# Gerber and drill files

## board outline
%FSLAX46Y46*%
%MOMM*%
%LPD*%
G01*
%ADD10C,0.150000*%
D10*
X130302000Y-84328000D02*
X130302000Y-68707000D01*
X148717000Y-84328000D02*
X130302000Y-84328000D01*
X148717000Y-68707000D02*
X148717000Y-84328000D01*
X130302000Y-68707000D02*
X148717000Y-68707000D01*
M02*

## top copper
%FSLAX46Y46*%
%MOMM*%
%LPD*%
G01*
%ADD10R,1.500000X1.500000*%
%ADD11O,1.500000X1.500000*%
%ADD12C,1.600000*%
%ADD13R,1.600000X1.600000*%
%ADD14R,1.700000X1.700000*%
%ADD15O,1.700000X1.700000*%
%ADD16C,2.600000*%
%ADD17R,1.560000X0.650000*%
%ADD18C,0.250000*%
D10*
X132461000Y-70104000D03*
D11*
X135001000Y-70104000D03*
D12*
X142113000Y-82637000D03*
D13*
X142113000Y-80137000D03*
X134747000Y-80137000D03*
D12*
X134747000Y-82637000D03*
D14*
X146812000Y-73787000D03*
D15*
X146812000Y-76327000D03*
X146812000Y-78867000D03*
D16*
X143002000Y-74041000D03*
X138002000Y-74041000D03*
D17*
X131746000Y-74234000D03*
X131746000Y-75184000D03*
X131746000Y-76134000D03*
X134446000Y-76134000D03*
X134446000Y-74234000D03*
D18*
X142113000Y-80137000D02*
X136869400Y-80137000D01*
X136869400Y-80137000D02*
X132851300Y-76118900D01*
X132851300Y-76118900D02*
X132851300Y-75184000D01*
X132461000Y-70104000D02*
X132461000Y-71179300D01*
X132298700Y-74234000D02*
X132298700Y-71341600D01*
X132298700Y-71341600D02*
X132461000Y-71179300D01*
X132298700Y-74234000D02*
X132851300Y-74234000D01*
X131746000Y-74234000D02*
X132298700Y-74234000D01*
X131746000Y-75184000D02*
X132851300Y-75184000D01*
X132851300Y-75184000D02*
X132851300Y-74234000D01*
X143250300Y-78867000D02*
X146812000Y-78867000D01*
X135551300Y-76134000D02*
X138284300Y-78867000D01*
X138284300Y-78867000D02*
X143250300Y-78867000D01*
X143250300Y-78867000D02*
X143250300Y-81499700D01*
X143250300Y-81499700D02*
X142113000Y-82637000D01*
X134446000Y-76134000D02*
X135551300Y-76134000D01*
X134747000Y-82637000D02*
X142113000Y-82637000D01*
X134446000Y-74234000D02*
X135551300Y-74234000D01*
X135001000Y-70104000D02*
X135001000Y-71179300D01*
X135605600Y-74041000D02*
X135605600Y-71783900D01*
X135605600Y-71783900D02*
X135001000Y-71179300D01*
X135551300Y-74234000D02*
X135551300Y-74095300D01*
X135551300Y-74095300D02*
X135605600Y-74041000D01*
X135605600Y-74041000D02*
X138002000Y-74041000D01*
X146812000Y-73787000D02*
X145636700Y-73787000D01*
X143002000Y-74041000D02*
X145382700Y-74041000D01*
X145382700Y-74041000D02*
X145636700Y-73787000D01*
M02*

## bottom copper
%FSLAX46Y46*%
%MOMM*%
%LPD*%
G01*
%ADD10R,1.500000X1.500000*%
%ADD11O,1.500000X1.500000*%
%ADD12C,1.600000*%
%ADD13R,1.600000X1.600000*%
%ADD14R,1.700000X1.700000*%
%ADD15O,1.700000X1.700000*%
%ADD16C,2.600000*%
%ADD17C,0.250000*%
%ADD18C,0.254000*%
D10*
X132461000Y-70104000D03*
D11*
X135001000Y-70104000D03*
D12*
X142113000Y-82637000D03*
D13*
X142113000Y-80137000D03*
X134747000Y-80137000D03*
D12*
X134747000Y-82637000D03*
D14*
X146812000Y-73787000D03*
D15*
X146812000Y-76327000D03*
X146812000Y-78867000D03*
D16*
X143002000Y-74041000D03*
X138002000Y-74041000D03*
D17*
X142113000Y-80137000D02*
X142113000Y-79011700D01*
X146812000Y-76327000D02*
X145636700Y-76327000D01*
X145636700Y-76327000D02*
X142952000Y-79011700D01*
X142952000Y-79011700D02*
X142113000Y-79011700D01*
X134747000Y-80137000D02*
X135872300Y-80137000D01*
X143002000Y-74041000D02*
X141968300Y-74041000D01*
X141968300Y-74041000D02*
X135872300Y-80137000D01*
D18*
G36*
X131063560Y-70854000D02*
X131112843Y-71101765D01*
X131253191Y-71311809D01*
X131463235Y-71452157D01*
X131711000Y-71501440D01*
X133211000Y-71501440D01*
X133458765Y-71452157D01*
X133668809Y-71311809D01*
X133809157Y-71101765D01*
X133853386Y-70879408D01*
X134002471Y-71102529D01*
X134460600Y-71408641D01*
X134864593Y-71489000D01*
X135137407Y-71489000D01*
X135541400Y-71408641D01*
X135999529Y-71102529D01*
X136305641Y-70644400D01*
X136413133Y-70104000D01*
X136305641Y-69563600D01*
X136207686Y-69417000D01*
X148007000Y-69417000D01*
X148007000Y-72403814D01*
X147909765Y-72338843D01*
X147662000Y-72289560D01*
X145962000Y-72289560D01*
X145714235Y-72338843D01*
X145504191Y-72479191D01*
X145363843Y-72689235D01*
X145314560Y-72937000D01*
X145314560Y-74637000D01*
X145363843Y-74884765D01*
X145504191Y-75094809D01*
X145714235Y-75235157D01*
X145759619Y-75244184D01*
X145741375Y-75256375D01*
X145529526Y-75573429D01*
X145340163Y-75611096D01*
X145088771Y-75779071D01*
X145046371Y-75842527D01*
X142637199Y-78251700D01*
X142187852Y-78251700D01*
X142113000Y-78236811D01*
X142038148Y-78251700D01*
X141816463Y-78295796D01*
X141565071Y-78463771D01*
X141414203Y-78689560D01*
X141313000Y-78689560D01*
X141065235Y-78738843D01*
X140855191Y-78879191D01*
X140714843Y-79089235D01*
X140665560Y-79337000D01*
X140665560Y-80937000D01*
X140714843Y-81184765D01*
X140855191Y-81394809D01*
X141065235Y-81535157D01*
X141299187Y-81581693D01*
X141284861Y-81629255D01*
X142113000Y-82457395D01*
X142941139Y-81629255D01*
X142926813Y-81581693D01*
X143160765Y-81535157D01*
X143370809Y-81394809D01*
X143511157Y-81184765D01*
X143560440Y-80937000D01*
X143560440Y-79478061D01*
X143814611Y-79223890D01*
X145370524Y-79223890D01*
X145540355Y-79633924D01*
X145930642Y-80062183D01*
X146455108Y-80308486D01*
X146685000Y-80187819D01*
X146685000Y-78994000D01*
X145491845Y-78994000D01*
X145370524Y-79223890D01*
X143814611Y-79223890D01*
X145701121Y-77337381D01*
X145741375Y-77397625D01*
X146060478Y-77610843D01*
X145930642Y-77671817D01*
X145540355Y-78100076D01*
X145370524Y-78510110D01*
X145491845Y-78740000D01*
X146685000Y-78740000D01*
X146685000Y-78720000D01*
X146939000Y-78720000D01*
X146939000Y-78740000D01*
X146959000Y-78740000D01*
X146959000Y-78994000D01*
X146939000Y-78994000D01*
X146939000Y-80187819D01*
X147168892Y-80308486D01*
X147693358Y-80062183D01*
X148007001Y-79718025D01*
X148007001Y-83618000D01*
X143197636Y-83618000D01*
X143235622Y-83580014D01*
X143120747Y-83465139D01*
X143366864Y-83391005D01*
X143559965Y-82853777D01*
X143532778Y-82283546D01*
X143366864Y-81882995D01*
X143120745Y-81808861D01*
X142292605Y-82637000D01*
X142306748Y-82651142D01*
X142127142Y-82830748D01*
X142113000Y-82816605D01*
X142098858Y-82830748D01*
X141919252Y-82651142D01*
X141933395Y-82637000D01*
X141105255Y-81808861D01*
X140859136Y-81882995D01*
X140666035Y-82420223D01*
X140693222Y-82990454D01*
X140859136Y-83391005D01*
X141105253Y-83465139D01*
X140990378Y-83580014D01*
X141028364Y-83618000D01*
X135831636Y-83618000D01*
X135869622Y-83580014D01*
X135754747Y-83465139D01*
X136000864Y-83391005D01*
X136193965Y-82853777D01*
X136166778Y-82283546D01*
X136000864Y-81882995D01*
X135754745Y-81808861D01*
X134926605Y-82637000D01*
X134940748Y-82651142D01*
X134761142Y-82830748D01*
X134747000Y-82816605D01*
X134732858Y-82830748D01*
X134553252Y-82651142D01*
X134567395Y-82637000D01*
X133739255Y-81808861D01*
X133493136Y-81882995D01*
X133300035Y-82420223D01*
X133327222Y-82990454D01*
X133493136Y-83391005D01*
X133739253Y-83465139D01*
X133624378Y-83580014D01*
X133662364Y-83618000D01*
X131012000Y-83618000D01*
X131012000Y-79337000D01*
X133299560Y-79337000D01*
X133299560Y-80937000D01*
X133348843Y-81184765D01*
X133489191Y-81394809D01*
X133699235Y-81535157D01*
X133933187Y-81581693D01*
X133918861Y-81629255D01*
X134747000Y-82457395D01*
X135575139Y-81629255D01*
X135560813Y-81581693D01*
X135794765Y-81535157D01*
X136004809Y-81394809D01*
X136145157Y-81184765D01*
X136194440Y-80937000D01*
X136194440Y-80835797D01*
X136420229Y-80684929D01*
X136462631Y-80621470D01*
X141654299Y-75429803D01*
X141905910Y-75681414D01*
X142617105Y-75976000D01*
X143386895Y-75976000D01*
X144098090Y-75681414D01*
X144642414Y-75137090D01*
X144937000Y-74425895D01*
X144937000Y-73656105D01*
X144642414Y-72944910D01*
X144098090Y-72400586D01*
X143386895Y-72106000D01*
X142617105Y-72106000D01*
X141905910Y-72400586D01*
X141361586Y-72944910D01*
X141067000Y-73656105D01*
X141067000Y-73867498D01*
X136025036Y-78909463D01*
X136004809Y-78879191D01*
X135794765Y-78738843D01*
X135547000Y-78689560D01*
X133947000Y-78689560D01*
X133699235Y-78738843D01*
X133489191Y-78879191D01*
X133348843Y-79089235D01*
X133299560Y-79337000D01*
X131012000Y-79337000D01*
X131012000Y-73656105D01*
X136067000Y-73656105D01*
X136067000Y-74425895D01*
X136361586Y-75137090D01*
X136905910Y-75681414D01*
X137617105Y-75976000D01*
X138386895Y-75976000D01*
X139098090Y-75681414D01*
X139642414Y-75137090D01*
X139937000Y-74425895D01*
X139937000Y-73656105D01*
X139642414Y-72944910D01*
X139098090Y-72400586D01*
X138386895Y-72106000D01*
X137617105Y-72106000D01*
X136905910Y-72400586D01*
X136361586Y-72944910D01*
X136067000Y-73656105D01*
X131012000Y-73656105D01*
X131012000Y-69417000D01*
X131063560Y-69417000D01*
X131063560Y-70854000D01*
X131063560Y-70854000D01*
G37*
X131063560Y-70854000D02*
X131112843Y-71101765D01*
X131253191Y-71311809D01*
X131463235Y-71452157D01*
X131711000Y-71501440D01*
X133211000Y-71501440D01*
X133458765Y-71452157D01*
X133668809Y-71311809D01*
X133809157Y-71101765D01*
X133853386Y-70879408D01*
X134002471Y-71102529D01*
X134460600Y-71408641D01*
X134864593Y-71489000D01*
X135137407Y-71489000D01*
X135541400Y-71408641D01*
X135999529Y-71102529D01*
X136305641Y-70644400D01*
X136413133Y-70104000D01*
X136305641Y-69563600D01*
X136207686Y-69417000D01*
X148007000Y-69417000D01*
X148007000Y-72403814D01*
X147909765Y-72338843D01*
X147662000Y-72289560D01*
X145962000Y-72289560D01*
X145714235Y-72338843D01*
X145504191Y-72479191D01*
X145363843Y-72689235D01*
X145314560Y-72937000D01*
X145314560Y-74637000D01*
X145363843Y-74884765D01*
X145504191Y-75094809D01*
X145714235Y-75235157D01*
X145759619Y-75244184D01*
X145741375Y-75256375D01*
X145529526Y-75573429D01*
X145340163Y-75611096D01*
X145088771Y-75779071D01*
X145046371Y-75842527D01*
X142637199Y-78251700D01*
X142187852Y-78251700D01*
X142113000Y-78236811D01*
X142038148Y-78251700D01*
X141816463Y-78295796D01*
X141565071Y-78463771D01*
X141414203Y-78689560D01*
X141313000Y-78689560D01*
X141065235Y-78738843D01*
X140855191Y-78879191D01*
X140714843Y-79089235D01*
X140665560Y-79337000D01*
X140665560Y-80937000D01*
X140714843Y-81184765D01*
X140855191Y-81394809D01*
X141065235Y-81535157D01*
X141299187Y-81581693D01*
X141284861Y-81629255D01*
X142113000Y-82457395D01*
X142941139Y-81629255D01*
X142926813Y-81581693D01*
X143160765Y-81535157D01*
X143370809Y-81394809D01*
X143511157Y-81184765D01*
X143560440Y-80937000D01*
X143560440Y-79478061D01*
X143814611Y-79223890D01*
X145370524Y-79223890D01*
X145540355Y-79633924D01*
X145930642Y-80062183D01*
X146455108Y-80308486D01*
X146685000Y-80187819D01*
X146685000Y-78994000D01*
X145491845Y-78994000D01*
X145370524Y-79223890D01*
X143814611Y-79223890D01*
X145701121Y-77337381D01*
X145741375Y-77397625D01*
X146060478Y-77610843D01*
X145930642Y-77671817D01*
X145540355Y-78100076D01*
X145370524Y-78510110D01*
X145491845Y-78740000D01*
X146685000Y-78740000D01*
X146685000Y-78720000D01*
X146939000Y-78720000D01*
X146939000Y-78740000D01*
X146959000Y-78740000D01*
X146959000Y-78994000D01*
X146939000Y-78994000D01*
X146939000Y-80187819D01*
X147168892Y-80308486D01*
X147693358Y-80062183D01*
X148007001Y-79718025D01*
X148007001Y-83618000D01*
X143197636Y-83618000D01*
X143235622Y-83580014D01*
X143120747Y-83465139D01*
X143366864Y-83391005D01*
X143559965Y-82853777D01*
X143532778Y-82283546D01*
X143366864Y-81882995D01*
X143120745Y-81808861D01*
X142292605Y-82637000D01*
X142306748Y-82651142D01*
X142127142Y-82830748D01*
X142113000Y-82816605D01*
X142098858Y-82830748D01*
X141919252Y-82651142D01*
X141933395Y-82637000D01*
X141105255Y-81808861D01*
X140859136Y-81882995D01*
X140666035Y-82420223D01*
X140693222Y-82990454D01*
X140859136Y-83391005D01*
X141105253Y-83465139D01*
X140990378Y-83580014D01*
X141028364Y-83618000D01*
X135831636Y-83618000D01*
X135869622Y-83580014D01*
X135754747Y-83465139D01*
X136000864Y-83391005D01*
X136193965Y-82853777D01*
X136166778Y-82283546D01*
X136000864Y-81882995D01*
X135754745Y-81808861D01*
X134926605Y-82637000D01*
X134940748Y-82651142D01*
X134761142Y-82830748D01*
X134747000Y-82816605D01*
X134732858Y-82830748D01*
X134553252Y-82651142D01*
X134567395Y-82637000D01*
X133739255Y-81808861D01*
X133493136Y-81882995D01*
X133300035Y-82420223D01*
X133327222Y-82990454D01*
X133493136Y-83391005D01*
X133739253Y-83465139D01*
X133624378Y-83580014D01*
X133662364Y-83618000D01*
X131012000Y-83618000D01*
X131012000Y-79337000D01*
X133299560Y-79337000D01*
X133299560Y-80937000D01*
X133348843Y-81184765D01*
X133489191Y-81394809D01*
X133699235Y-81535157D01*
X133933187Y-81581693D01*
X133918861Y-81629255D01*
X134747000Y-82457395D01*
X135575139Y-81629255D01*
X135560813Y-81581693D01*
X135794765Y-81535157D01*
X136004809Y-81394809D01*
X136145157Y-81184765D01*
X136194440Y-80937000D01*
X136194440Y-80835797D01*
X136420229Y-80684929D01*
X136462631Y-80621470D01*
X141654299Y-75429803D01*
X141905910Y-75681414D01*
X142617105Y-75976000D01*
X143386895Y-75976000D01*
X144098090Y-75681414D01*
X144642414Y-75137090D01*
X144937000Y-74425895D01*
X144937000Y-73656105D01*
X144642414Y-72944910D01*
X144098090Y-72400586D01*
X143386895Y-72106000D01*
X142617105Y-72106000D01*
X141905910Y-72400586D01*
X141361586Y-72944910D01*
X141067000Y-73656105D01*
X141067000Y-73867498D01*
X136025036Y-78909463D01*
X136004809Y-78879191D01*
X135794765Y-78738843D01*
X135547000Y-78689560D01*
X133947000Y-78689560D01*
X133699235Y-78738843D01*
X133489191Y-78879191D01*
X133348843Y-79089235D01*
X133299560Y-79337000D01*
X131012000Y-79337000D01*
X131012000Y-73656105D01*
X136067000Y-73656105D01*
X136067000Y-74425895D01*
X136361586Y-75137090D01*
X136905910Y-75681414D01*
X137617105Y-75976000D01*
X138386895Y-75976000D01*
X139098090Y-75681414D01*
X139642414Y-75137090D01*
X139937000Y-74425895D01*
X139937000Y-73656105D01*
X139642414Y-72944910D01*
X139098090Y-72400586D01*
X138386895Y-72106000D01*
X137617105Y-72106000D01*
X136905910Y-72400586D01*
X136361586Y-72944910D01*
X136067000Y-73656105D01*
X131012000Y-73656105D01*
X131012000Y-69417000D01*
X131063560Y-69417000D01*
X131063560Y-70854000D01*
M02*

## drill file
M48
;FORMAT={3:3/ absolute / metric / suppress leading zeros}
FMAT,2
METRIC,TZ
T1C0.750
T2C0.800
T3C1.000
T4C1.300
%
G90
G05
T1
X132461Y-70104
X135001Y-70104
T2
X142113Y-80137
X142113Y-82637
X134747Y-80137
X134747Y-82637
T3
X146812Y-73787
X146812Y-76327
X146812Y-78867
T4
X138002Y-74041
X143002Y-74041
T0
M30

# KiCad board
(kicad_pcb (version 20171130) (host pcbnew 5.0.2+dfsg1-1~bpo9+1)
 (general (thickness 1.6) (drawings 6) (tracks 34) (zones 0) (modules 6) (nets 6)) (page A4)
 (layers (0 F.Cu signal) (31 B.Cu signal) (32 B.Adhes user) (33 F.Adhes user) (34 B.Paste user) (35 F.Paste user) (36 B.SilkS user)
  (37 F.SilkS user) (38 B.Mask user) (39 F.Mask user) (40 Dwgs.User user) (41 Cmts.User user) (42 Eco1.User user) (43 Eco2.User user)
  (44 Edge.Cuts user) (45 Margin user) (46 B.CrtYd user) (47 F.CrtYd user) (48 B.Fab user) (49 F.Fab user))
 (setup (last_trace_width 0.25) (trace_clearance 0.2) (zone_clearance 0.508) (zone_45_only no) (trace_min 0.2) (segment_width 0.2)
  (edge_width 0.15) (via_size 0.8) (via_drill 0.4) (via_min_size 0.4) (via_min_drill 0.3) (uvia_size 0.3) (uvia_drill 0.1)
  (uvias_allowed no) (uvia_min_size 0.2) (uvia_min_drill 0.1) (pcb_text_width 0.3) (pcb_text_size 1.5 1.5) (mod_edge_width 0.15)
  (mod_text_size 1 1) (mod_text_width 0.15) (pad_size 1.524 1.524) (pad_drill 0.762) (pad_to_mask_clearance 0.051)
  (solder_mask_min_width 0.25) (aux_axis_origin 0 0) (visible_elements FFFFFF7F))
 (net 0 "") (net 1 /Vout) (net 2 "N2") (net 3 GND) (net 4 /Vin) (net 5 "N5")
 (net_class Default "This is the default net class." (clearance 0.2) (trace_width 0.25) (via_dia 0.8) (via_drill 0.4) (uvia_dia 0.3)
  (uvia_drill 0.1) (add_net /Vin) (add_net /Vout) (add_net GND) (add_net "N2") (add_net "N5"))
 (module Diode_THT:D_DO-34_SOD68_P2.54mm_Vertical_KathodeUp (layer F.Cu) (at 132.461 70.104)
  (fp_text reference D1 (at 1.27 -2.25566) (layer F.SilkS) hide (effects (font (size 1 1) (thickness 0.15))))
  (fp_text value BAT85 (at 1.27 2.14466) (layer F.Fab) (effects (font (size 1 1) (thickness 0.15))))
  (pad 1 thru_hole rect (at 0 0) (size 1.5 1.5) (drill 0.75) (layers *.Cu *.Mask) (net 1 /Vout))
  (pad 2 thru_hole oval (at 2.54 0) (size 1.5 1.5) (drill 0.75) (layers *.Cu *.Mask) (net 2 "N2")))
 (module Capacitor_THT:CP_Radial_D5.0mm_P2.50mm (layer F.Cu) (at 142.113 80.137 270)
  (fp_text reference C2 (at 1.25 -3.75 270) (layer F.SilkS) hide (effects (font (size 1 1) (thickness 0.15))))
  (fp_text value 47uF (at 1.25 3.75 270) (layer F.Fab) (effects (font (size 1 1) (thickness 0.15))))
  (pad 2 thru_hole circle (at 2.5 0 270) (size 1.6 1.6) (drill 0.8) (layers *.Cu *.Mask) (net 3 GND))
  (pad 1 thru_hole rect (at 0 0 270) (size 1.6 1.6) (drill 0.8) (layers *.Cu *.Mask) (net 1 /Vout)))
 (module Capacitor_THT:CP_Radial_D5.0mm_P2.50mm (layer F.Cu) (at 134.747 80.137 270)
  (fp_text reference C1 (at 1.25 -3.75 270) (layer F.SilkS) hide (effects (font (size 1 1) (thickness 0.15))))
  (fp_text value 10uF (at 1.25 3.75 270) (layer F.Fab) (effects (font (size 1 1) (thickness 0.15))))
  (pad 1 thru_hole rect (at 0 0 270) (size 1.6 1.6) (drill 0.8) (layers *.Cu *.Mask) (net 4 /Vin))
  (pad 2 thru_hole circle (at 2.5 0 270) (size 1.6 1.6) (drill 0.8) (layers *.Cu *.Mask) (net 3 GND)))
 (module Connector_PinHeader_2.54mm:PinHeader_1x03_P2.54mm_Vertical (layer F.Cu) (at 146.812 73.787)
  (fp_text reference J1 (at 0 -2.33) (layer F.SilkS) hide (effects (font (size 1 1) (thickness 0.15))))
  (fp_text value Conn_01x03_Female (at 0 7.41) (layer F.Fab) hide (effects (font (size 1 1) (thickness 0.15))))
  (pad 1 thru_hole rect (at 0 0) (size 1.7 1.7) (drill 1) (layers *.Cu *.Mask) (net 4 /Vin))
  (pad 2 thru_hole oval (at 0 2.54) (size 1.7 1.7) (drill 1) (layers *.Cu *.Mask) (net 1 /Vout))
  (pad 3 thru_hole oval (at 0 5.08) (size 1.7 1.7) (drill 1) (layers *.Cu *.Mask) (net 3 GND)))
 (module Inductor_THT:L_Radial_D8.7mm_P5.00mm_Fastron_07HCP (layer F.Cu) (at 143.002 74.041 180)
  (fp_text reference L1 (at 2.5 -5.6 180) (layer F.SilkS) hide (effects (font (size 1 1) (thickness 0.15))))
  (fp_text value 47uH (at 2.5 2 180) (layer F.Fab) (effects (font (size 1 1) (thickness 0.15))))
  (pad 1 thru_hole circle (at 0 0 180) (size 2.6 2.6) (drill 1.3) (layers *.Cu *.Mask) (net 4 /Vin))
  (pad 2 thru_hole circle (at 5 0 180) (size 2.6 2.6) (drill 1.3) (layers *.Cu *.Mask) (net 2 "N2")))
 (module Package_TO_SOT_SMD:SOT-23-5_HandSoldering (layer F.Cu) (at 133.096 75.184)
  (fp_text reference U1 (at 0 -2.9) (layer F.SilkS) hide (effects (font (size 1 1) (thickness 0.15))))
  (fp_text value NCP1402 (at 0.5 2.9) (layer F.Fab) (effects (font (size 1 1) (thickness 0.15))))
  (pad 1 smd rect (at -1.35 -0.95) (size 1.56 0.65) (layers F.Cu F.Paste F.Mask) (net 1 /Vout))
  (pad 2 smd rect (at -1.35 0) (size 1.56 0.65) (layers F.Cu F.Paste F.Mask) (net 1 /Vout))
  (pad 3 smd rect (at -1.35 0.95) (size 1.56 0.65) (layers F.Cu F.Paste F.Mask) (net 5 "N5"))
  (pad 4 smd rect (at 1.35 0.95) (size 1.56 0.65) (layers F.Cu F.Paste F.Mask) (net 3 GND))
  (pad 5 smd rect (at 1.35 -0.95) (size 1.56 0.65) (layers F.Cu F.Paste F.Mask) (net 2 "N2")))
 (gr_line (start 130.302 84.328) (end 130.302 68.707) (layer Edge.Cuts) (width 0.15))
 (gr_line (start 148.717 84.328) (end 130.302 84.328) (layer Edge.Cuts) (width 0.15))
 (gr_line (start 148.717 68.707) (end 148.717 84.328) (layer Edge.Cuts) (width 0.15))
 (gr_line (start 130.302 68.707) (end 148.717 68.707) (layer Edge.Cuts) (width 0.15))
 (segment (start 142.113 80.137) (end 136.8694 80.137) (width 0.25) (layer F.Cu) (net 1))
 (segment (start 136.8694 80.137) (end 132.8513 76.1189) (width 0.25) (layer F.Cu) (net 1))
 (segment (start 132.8513 76.1189) (end 132.8513 75.184) (width 0.25) (layer F.Cu) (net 1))
 (segment (start 142.113 80.137) (end 142.113 79.0117) (width 0.25) (layer B.Cu) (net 1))
 (segment (start 146.812 76.327) (end 145.6367 76.327) (width 0.25) (layer B.Cu) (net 1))
 (segment (start 145.6367 76.327) (end 142.952 79.0117) (width 0.25) (layer B.Cu) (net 1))
 (segment (start 142.952 79.0117) (end 142.113 79.0117) (width 0.25) (layer B.Cu) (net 1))
 (segment (start 132.461 70.104) (end 132.461 71.1793) (width 0.25) (layer F.Cu) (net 1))
 (segment (start 132.2987 74.234) (end 132.2987 71.3416) (width 0.25) (layer F.Cu) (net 1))
 (segment (start 132.2987 71.3416) (end 132.461 71.1793) (width 0.25) (layer F.Cu) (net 1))
 (segment (start 132.2987 74.234) (end 132.8513 74.234) (width 0.25) (layer F.Cu) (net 1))
 (segment (start 131.746 74.234) (end 132.2987 74.234) (width 0.25) (layer F.Cu) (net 1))
 (segment (start 131.746 75.184) (end 132.8513 75.184) (width 0.25) (layer F.Cu) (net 1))
 (segment (start 132.8513 75.184) (end 132.8513 74.234) (width 0.25) (layer F.Cu) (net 1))
 (segment (start 143.2503 78.867) (end 146.812 78.867) (width 0.25) (layer F.Cu) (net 3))
 (segment (start 135.5513 76.134) (end 138.2843 78.867) (width 0.25) (layer F.Cu) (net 3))
 (segment (start 138.2843 78.867) (end 143.2503 78.867) (width 0.25) (layer F.Cu) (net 3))
 (segment (start 143.2503 78.867) (end 143.2503 81.4997) (width 0.25) (layer F.Cu) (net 3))
 (segment (start 143.2503 81.4997) (end 142.113 82.637) (width 0.25) (layer F.Cu) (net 3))
 (segment (start 134.446 76.134) (end 135.5513 76.134) (width 0.25) (layer F.Cu) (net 3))
 (segment (start 134.747 82.637) (end 142.113 82.637) (width 0.25) (layer F.Cu) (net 3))
 (segment (start 134.446 74.234) (end 135.5513 74.234) (width 0.25) (layer F.Cu) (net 2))
 (segment (start 135.001 70.104) (end 135.001 71.1793) (width 0.25) (layer F.Cu) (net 2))
 (segment (start 135.6056 74.041) (end 135.6056 71.7839) (width 0.25) (layer F.Cu) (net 2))
 (segment (start 135.6056 71.7839) (end 135.001 71.1793) (width 0.25) (layer F.Cu) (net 2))
 (segment (start 135.5513 74.234) (end 135.5513 74.0953) (width 0.25) (layer F.Cu) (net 2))
 (segment (start 135.5513 74.0953) (end 135.6056 74.041) (width 0.25) (layer F.Cu) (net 2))
 (segment (start 135.6056 74.041) (end 138.002 74.041) (width 0.25) (layer F.Cu) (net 2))
 (segment (start 134.747 80.137) (end 135.8723 80.137) (width 0.25) (layer B.Cu) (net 4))
 (segment (start 143.002 74.041) (end 141.9683 74.041) (width 0.25) (layer B.Cu) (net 4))
 (segment (start 141.9683 74.041) (end 135.8723 80.137) (width 0.25) (layer B.Cu) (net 4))
 (segment (start 146.812 73.787) (end 145.6367 73.787) (width 0.25) (layer F.Cu) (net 4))
 (segment (start 143.002 74.041) (end 145.3827 74.041) (width 0.25) (layer F.Cu) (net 4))
 (segment (start 145.3827 74.041) (end 145.6367 73.787) (width 0.25) (layer F.Cu) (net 4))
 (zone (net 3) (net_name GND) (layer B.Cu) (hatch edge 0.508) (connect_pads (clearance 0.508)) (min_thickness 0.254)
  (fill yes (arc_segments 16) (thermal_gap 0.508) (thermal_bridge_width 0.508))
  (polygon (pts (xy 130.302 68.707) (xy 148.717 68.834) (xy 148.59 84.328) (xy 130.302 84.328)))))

